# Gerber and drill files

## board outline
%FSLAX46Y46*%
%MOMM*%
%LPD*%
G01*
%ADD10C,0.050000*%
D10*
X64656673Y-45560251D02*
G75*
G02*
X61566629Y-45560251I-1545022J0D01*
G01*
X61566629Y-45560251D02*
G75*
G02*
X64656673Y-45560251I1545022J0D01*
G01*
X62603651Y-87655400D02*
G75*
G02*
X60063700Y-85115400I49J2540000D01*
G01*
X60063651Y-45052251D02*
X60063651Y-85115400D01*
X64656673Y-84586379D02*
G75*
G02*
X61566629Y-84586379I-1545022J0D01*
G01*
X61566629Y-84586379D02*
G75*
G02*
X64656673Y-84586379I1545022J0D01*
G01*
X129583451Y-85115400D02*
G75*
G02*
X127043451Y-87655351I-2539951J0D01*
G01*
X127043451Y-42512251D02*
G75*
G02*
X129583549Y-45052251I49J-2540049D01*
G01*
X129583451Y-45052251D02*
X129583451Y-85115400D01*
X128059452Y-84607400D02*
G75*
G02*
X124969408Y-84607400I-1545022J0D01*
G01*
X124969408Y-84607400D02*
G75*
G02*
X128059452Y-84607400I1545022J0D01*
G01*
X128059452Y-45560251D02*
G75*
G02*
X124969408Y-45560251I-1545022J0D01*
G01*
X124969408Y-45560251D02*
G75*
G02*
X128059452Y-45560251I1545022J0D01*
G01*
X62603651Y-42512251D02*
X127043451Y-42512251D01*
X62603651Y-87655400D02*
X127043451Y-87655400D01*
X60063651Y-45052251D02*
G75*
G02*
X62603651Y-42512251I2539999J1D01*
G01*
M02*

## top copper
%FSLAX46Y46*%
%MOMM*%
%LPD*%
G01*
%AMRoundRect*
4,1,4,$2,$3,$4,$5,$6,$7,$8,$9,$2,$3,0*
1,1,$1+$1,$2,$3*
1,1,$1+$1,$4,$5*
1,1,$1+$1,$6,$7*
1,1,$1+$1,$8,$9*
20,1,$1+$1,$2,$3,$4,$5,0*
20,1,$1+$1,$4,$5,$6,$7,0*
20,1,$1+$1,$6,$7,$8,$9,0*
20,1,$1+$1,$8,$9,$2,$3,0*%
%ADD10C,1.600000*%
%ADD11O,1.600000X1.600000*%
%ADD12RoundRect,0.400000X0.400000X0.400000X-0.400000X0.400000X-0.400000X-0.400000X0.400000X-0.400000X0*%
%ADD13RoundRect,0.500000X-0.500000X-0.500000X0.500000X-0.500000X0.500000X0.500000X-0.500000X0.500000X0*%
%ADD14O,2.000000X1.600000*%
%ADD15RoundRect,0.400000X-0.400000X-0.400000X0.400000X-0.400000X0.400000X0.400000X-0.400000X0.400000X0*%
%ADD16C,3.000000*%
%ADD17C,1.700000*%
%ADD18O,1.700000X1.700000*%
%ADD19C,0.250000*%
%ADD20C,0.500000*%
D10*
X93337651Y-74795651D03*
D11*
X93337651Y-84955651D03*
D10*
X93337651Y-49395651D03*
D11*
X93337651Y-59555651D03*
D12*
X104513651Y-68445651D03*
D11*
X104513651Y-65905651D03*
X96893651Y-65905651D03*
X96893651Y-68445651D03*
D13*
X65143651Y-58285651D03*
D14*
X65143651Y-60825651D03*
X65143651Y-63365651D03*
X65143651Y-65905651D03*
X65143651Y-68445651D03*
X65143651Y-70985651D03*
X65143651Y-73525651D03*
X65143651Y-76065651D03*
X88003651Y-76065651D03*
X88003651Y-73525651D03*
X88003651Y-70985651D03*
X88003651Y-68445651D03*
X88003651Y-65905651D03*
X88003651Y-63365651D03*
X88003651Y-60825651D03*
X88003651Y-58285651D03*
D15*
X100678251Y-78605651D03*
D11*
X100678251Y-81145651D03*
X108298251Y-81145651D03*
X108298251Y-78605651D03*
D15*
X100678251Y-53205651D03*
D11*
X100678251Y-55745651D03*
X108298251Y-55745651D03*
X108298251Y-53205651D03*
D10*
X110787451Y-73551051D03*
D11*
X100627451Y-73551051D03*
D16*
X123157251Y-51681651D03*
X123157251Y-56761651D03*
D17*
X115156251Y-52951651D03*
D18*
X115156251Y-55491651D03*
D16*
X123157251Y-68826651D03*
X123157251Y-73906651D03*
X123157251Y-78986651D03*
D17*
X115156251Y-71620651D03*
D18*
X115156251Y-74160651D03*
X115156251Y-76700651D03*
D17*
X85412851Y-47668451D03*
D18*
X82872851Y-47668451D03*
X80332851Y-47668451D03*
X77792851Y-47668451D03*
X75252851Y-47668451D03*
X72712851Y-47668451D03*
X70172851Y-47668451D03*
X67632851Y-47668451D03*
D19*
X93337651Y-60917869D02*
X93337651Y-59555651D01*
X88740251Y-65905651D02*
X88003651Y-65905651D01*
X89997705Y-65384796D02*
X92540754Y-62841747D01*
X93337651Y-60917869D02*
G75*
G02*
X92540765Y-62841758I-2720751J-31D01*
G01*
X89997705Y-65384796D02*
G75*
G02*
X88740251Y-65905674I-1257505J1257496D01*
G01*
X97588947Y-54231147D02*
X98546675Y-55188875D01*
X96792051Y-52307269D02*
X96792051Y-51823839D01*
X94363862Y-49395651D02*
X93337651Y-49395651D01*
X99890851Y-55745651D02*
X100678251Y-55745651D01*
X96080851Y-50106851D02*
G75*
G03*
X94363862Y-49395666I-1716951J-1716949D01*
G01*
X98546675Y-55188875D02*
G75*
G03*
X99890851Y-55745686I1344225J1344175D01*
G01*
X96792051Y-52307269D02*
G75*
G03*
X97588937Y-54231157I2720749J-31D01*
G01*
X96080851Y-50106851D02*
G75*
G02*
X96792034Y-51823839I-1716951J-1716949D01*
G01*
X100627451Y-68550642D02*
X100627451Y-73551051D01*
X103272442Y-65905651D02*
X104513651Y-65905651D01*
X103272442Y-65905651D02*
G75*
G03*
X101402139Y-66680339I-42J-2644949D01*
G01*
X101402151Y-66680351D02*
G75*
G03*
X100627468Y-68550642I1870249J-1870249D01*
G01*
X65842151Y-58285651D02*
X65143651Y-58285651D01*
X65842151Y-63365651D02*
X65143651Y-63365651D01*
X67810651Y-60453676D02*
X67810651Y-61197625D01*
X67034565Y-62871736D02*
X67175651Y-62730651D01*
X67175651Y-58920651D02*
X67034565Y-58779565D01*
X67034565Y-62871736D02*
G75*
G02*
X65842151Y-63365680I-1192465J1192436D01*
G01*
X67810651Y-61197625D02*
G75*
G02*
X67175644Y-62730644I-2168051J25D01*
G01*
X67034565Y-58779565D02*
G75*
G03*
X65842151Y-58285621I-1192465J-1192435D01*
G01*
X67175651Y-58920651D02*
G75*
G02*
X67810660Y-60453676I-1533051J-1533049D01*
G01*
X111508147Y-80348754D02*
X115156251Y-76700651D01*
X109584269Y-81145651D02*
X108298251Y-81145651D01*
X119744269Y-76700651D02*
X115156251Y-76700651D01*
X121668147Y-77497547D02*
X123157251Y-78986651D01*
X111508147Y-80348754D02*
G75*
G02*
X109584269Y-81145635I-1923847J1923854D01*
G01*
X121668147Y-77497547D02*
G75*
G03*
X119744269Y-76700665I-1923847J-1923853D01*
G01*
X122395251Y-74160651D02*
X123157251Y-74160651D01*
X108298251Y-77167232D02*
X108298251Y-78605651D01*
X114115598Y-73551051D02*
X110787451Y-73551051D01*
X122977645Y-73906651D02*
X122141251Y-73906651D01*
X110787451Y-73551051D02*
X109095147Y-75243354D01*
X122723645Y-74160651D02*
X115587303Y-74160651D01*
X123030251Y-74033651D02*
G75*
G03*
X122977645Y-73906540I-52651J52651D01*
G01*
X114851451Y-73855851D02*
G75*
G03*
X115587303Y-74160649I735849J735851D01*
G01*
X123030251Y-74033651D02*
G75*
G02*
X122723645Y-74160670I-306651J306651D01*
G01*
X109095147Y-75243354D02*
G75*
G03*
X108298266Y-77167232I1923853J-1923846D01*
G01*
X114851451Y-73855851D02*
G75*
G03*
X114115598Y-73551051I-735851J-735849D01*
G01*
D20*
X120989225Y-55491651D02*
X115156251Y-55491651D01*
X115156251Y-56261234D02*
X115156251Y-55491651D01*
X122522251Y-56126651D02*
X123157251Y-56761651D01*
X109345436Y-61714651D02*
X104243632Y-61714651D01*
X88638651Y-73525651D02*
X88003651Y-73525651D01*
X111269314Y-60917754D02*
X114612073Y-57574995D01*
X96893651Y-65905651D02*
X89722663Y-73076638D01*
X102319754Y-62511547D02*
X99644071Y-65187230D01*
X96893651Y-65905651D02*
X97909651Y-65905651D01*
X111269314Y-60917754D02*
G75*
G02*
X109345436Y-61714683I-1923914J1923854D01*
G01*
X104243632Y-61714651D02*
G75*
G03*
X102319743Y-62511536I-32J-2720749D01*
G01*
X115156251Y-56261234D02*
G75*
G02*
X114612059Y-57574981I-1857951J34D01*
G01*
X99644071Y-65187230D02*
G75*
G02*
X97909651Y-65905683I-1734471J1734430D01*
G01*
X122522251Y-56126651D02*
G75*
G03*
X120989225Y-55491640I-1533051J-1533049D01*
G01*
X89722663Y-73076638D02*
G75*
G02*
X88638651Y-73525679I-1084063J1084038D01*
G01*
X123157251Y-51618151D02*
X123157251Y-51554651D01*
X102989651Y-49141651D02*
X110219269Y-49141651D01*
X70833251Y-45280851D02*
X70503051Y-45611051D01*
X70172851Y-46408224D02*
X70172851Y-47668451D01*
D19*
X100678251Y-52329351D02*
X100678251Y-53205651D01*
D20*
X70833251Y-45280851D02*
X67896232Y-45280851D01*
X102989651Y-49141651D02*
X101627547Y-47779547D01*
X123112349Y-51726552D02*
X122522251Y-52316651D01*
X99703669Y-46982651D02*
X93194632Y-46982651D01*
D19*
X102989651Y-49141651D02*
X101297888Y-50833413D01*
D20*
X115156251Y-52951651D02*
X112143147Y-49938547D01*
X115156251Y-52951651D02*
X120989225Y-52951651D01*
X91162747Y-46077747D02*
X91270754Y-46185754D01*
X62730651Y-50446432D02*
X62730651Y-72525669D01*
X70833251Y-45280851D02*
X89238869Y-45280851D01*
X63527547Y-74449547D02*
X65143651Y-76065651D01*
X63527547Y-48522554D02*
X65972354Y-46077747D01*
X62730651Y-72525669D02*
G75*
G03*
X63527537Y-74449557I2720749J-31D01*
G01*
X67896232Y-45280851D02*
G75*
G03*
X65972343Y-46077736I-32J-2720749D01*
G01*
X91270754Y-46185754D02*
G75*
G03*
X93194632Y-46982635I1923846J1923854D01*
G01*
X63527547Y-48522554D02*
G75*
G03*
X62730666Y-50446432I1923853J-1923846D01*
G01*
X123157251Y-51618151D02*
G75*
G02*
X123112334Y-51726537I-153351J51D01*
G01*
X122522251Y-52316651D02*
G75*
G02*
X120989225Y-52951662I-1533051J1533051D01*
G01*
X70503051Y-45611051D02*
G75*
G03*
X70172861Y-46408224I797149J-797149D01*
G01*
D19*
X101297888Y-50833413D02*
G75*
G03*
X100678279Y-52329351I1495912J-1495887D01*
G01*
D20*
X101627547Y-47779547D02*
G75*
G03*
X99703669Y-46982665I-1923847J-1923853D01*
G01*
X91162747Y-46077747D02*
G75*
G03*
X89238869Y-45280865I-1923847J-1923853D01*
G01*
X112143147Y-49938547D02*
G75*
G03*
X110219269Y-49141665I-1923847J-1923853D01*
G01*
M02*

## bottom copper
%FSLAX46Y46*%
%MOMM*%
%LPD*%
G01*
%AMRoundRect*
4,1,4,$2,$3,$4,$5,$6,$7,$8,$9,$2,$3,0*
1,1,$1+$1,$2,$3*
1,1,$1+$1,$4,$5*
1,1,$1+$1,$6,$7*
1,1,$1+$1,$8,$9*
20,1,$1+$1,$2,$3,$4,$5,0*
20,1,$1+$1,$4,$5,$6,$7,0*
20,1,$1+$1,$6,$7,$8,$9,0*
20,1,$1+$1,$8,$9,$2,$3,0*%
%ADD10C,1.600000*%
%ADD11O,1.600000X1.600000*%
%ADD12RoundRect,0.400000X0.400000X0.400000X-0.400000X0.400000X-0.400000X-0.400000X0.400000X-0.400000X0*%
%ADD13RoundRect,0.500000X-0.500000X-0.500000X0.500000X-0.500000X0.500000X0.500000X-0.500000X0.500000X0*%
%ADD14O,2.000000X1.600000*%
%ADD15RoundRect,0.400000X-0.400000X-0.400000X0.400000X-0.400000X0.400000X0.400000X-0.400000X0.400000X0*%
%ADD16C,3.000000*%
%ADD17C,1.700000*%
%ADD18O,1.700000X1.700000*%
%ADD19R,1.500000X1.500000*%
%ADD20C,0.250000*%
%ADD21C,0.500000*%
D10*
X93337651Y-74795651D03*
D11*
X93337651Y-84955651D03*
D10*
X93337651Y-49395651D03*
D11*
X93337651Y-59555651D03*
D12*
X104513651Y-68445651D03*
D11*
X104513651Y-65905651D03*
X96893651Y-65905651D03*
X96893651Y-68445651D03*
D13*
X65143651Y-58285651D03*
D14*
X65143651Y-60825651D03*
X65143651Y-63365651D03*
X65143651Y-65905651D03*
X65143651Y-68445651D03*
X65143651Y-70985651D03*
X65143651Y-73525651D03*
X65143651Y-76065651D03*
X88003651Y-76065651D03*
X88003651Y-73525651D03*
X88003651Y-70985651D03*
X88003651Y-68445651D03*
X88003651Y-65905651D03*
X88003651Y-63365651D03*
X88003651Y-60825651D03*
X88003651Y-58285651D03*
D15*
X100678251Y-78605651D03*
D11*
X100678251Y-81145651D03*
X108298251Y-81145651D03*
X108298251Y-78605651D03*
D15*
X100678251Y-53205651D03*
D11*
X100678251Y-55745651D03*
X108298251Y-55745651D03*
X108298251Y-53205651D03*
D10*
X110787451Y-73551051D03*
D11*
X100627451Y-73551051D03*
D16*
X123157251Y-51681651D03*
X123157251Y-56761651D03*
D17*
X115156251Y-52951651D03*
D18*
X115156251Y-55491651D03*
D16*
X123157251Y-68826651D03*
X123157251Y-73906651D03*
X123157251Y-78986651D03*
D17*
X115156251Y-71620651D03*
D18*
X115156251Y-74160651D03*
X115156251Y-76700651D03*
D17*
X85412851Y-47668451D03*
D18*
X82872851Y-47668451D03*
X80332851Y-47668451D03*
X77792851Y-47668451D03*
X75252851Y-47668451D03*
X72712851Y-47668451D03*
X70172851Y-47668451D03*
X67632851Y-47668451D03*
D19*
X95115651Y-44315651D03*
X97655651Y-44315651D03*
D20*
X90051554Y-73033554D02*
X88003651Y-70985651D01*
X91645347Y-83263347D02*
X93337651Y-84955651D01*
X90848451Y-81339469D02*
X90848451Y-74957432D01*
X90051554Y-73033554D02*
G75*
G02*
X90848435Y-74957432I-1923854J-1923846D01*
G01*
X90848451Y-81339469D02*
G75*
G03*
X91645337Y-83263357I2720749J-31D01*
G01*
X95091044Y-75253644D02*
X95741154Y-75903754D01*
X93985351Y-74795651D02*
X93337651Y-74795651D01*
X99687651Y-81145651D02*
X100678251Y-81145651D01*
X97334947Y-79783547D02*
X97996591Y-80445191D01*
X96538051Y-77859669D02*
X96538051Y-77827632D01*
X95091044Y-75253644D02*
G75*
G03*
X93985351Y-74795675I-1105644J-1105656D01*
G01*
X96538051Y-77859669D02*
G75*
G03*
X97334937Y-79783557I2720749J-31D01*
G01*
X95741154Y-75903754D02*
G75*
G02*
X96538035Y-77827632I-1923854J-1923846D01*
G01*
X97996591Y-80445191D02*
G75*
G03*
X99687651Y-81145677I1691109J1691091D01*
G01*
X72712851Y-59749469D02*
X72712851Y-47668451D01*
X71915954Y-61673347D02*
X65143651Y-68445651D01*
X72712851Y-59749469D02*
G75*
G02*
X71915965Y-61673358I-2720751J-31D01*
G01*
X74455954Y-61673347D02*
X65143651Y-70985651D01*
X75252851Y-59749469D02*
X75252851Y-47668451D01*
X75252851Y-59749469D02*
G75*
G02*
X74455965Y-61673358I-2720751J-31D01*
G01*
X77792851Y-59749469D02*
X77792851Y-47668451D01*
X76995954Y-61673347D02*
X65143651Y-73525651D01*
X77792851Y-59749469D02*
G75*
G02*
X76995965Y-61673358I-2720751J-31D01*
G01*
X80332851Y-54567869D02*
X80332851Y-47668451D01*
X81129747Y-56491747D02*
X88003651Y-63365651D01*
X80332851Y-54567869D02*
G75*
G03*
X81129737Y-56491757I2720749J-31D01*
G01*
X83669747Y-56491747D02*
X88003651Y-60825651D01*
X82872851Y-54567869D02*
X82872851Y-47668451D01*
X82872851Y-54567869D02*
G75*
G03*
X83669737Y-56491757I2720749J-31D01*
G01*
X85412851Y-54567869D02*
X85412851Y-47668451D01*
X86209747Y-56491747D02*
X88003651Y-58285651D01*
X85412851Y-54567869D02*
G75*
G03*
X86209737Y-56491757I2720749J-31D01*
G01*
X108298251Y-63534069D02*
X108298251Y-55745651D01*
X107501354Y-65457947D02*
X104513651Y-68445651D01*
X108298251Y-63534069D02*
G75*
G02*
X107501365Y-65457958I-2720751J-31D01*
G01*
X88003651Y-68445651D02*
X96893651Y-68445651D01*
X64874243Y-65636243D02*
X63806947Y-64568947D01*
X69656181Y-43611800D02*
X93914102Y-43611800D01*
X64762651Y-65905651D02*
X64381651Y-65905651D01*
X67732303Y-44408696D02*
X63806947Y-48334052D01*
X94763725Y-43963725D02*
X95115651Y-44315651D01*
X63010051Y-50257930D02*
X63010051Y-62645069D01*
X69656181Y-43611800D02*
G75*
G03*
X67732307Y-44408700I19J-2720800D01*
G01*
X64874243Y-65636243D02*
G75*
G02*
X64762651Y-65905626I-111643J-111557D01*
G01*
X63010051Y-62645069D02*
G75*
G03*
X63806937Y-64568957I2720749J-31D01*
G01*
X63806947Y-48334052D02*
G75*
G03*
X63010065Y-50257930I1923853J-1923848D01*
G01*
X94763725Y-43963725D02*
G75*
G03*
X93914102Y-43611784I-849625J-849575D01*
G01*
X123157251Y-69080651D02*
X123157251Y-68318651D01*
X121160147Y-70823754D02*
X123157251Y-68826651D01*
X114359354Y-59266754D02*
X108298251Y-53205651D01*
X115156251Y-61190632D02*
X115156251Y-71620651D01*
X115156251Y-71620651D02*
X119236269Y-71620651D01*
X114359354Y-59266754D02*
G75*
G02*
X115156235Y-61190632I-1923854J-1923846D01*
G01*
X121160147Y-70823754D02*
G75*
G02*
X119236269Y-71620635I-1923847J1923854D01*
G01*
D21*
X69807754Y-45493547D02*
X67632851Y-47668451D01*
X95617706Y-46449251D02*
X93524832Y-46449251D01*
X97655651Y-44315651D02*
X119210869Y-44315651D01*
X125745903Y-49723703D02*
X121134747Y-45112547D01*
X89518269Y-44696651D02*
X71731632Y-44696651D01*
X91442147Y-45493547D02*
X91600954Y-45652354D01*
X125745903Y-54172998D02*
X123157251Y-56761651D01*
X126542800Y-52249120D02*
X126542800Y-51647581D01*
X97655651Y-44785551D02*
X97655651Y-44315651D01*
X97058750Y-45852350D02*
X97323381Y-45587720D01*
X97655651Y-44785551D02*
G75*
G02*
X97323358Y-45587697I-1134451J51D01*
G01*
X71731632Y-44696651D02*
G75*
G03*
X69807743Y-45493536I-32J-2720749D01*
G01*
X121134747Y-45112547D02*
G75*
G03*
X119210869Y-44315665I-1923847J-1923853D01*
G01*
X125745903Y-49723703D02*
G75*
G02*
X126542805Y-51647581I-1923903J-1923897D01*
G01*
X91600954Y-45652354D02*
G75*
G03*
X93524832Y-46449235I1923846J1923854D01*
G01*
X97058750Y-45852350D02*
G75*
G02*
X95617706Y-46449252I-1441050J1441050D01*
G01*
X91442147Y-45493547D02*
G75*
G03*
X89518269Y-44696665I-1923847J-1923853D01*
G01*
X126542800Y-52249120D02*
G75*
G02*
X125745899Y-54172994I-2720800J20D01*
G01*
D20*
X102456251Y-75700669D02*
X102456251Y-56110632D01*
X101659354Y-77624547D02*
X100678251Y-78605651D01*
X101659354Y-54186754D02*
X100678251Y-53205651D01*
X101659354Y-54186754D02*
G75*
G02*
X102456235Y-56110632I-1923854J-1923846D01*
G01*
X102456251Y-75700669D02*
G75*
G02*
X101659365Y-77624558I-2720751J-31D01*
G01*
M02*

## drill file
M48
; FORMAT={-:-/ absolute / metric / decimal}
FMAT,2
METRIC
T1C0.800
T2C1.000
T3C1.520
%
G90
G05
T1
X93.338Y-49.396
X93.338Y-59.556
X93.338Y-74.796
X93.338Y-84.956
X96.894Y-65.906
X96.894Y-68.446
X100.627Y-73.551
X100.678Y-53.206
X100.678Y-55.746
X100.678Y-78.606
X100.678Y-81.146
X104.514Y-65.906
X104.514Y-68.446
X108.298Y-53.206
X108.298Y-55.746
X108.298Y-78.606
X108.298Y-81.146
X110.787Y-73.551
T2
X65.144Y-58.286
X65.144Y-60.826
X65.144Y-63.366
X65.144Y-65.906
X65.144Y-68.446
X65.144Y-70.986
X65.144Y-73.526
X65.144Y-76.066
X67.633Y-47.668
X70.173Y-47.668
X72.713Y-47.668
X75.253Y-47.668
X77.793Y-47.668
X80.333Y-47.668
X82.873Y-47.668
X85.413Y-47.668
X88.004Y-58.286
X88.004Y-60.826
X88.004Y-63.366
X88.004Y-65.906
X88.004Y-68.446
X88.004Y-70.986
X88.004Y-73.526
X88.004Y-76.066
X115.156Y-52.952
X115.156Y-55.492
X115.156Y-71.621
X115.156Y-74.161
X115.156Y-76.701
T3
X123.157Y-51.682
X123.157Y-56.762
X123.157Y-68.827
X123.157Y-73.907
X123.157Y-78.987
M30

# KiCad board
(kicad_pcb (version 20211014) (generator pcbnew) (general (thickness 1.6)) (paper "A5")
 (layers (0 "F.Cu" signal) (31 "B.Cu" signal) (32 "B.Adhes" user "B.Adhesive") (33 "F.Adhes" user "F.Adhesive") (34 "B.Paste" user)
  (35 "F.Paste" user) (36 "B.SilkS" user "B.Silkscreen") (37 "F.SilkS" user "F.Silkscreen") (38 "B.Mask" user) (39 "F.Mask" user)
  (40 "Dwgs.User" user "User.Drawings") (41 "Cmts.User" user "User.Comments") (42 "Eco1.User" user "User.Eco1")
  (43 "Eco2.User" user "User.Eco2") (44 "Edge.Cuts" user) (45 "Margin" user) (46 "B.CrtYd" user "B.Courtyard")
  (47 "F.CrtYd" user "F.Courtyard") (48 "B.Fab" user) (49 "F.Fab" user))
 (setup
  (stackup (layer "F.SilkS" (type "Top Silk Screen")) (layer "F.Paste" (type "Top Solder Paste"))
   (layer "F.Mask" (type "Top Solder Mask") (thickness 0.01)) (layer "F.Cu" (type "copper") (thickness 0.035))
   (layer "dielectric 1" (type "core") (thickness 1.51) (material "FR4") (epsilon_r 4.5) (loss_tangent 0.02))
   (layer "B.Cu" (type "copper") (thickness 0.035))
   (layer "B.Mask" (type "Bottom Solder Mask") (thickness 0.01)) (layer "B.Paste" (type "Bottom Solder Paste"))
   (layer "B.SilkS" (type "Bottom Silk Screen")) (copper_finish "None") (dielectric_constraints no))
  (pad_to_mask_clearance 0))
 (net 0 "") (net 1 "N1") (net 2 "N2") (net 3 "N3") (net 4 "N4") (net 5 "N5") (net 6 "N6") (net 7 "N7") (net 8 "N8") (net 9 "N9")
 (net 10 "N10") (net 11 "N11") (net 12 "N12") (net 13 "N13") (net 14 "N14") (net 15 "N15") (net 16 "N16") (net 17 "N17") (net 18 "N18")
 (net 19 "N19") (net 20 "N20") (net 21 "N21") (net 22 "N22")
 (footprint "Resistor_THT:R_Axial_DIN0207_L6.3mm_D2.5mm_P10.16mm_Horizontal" (layer "F.Cu") (at 93.337651 74.795651 -90)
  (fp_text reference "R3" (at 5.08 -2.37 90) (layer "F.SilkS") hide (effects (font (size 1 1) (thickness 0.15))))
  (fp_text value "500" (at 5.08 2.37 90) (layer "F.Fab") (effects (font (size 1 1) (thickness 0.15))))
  (pad "1" thru_hole circle locked (at 0 0 270) (size 1.6 1.6) (drill 0.8) (layers *.Cu *.Mask) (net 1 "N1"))
  (pad "2" thru_hole oval locked (at 10.16 0 270) (size 1.6 1.6) (drill 0.8) (layers *.Cu *.Mask) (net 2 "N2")))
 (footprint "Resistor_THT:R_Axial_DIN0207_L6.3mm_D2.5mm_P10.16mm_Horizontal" (layer "F.Cu") (at 93.337651 49.395651 -90)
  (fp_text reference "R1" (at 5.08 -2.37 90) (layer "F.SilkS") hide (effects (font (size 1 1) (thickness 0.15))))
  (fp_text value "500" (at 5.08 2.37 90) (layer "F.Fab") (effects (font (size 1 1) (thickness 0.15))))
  (pad "1" thru_hole circle locked (at 0 0 270) (size 1.6 1.6) (drill 0.8) (layers *.Cu *.Mask) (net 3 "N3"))
  (pad "2" thru_hole oval locked (at 10.16 0 270) (size 1.6 1.6) (drill 0.8) (layers *.Cu *.Mask) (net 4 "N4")))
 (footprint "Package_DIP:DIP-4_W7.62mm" (layer "F.Cu") (at 104.513651 68.445651 180)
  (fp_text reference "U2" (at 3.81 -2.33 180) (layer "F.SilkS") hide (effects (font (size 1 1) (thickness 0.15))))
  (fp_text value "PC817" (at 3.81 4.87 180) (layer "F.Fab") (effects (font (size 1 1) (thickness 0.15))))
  (pad "1" thru_hole roundrect locked (at 0 0 180) (size 1.6 1.6) (drill 0.8) (layers *.Cu *.Mask) (roundrect_rratio 0.25) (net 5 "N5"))
  (pad "2" thru_hole oval locked (at 0 2.54 180) (size 1.6 1.6) (drill 0.8) (layers *.Cu *.Mask) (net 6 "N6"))
  (pad "3" thru_hole oval locked (at 7.62 2.54 180) (size 1.6 1.6) (drill 0.8) (layers *.Cu *.Mask) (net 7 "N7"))
  (pad "4" thru_hole oval locked (at 7.62 0 180) (size 1.6 1.6) (drill 0.8) (layers *.Cu *.Mask) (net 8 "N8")))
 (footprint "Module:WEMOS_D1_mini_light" (layer "F.Cu") (at 65.143651 58.285651)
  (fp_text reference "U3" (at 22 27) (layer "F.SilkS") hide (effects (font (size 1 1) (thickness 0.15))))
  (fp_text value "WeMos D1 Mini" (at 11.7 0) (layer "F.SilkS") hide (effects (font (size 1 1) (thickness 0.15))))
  (pad "1" thru_hole roundrect locked (at 0 0) (size 2 2) (drill 1) (layers *.Cu *.Mask) (roundrect_rratio 0.25) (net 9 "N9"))
  (pad "2" thru_hole oval locked (at 0 2.54) (size 2 1.6) (drill 1) (layers *.Cu *.Mask) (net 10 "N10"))
  (pad "3" thru_hole oval locked (at 0 5.08) (size 2 1.6) (drill 1) (layers *.Cu *.Mask) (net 9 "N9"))
  (pad "4" thru_hole oval locked (at 0 7.62) (size 2 1.6) (drill 1) (layers *.Cu *.Mask) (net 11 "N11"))
  (pad "5" thru_hole oval locked (at 0 10.16) (size 2 1.6) (drill 1) (layers *.Cu *.Mask) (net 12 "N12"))
  (pad "6" thru_hole oval locked (at 0 12.7) (size 2 1.6) (drill 1) (layers *.Cu *.Mask) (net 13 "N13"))
  (pad "7" thru_hole oval locked (at 0 15.24) (size 2 1.6) (drill 1) (layers *.Cu *.Mask) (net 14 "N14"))
  (pad "8" thru_hole oval locked (at 0 17.78) (size 2 1.6) (drill 1) (layers *.Cu *.Mask) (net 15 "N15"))
  (pad "9" thru_hole oval locked (at 22.86 17.78) (size 2 1.6) (drill 1) (layers *.Cu *.Mask) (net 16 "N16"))
  (pad "10" thru_hole oval locked (at 22.86 15.24) (size 2 1.6) (drill 1) (layers *.Cu *.Mask) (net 7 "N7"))
  (pad "11" thru_hole oval locked (at 22.86 12.7) (size 2 1.6) (drill 1) (layers *.Cu *.Mask) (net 2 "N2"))
  (pad "12" thru_hole oval locked (at 22.86 10.16) (size 2 1.6) (drill 1) (layers *.Cu *.Mask) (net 8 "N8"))
  (pad "13" thru_hole oval locked (at 22.86 7.62) (size 2 1.6) (drill 1) (layers *.Cu *.Mask) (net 4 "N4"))
  (pad "14" thru_hole oval locked (at 22.86 5.08) (size 2 1.6) (drill 1) (layers *.Cu *.Mask) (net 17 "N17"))
  (pad "15" thru_hole oval locked (at 22.86 2.54) (size 2 1.6) (drill 1) (layers *.Cu *.Mask) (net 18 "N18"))
  (pad "16" thru_hole oval locked (at 22.86 0) (size 2 1.6) (drill 1) (layers *.Cu *.Mask) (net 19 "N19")))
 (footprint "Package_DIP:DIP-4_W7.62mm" (layer "F.Cu") (at 100.678251 78.605651)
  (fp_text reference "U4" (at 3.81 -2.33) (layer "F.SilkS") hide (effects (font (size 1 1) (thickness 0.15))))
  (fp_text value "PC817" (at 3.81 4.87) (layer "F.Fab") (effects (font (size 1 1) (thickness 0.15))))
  (pad "1" thru_hole roundrect locked (at 0 0) (size 1.6 1.6) (drill 0.8) (layers *.Cu *.Mask) (roundrect_rratio 0.25) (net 15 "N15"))
  (pad "2" thru_hole oval locked (at 0 2.54) (size 1.6 1.6) (drill 0.8) (layers *.Cu *.Mask) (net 1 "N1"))
  (pad "3" thru_hole oval locked (at 7.62 2.54) (size 1.6 1.6) (drill 0.8) (layers *.Cu *.Mask) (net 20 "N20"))
  (pad "4" thru_hole oval locked (at 7.62 0) (size 1.6 1.6) (drill 0.8) (layers *.Cu *.Mask) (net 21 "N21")))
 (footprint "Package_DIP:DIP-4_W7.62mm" (layer "F.Cu") (at 100.678251 53.205651)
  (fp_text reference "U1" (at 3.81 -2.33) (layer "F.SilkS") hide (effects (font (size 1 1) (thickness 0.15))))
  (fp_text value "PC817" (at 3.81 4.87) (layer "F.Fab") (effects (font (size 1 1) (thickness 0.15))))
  (pad "1" thru_hole roundrect locked (at 0 0) (size 1.6 1.6) (drill 0.8) (layers *.Cu *.Mask) (roundrect_rratio 0.25) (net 15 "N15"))
  (pad "2" thru_hole oval locked (at 0 2.54) (size 1.6 1.6) (drill 0.8) (layers *.Cu *.Mask) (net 3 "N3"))
  (pad "3" thru_hole oval locked (at 7.62 2.54) (size 1.6 1.6) (drill 0.8) (layers *.Cu *.Mask) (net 5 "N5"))
  (pad "4" thru_hole oval locked (at 7.62 0) (size 1.6 1.6) (drill 0.8) (layers *.Cu *.Mask) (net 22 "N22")))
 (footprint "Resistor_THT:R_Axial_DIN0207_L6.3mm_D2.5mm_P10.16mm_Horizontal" (layer "F.Cu") (at 110.787451 73.551051 180)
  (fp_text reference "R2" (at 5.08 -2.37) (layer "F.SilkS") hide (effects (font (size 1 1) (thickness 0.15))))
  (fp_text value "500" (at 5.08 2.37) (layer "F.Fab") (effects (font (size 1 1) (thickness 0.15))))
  (pad "1" thru_hole circle locked (at 0 0 180) (size 1.6 1.6) (drill 0.8) (layers *.Cu *.Mask) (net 21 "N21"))
  (pad "2" thru_hole oval locked (at 10.16 0 180) (size 1.6 1.6) (drill 0.8) (layers *.Cu *.Mask) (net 6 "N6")))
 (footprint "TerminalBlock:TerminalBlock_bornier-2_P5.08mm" (layer "F.Cu") (at 123.157251 51.681651 -90)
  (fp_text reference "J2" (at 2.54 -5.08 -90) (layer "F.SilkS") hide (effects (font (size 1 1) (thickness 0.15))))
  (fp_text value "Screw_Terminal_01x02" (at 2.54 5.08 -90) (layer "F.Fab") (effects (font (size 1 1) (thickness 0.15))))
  (pad "1" thru_hole circle locked (at 0 0 270) (size 3 3) (drill 1.52) (layers *.Cu *.Mask) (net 15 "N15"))
  (pad "2" thru_hole circle locked (at 5.08 0 270) (size 3 3) (drill 1.52) (layers *.Cu *.Mask) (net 7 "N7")))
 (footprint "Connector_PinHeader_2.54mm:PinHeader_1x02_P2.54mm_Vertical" (layer "F.Cu") (at 115.156251 52.951651)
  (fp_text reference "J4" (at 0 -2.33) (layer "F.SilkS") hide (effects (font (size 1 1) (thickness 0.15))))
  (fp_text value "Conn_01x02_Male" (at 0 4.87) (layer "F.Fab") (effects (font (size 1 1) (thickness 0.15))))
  (pad "1" thru_hole circle locked (at 0 0) (size 1.7 1.7) (drill 1) (layers *.Cu *.Mask) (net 15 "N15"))
  (pad "2" thru_hole oval locked (at 0 2.54) (size 1.7 1.7) (drill 1) (layers *.Cu *.Mask) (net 7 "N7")))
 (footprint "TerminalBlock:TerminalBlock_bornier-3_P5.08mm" (layer "F.Cu") (at 123.157251 68.826651 -90)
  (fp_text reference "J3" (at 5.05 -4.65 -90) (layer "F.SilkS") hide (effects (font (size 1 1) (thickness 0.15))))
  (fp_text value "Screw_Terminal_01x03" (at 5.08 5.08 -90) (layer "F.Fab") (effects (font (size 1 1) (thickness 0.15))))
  (pad "1" thru_hole circle locked (at 0 0 270) (size 3 3) (drill 1.52) (layers *.Cu *.Mask) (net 22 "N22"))
  (pad "2" thru_hole circle locked (at 5.08 0 270) (size 3 3) (drill 1.52) (layers *.Cu *.Mask) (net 21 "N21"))
  (pad "3" thru_hole circle locked (at 10.16 0 270) (size 3 3) (drill 1.52) (layers *.Cu *.Mask) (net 20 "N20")))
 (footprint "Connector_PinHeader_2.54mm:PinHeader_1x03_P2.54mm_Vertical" (layer "F.Cu") (at 115.156251 71.620651)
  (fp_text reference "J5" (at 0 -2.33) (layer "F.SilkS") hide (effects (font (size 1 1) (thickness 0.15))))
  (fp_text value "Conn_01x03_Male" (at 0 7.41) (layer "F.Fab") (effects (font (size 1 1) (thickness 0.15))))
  (pad "1" thru_hole circle locked (at 0 0) (size 1.7 1.7) (drill 1) (layers *.Cu *.Mask) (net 22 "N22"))
  (pad "2" thru_hole oval locked (at 0 2.54) (size 1.7 1.7) (drill 1) (layers *.Cu *.Mask) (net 21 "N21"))
  (pad "3" thru_hole oval locked (at 0 5.08) (size 1.7 1.7) (drill 1) (layers *.Cu *.Mask) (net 20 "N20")))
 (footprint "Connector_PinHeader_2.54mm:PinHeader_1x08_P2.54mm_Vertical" (layer "F.Cu") (at 85.412851 47.668451 -90)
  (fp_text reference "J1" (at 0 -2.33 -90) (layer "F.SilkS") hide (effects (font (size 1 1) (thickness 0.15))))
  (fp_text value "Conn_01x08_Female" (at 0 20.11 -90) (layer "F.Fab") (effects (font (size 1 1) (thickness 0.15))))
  (pad "1" thru_hole circle locked (at 0 0 270) (size 1.7 1.7) (drill 1) (layers *.Cu *.Mask) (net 19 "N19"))
  (pad "2" thru_hole oval locked (at 0 2.54 270) (size 1.7 1.7) (drill 1) (layers *.Cu *.Mask) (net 18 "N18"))
  (pad "3" thru_hole oval locked (at 0 5.08 270) (size 1.7 1.7) (drill 1) (layers *.Cu *.Mask) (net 17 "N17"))
  (pad "4" thru_hole oval locked (at 0 7.62 270) (size 1.7 1.7) (drill 1) (layers *.Cu *.Mask) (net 14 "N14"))
  (pad "5" thru_hole oval locked (at 0 10.16 270) (size 1.7 1.7) (drill 1) (layers *.Cu *.Mask) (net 13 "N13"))
  (pad "6" thru_hole oval locked (at 0 12.7 270) (size 1.7 1.7) (drill 1) (layers *.Cu *.Mask) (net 12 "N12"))
  (pad "7" thru_hole oval locked (at 0 15.24 270) (size 1.7 1.7) (drill 1) (layers *.Cu *.Mask) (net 15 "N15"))
  (pad "8" thru_hole oval locked (at 0 17.78 270) (size 1.7 1.7) (drill 1) (layers *.Cu *.Mask) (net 7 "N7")))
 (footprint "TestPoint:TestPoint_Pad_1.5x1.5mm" (layer "B.Cu") (at 95.115651 44.315651 180)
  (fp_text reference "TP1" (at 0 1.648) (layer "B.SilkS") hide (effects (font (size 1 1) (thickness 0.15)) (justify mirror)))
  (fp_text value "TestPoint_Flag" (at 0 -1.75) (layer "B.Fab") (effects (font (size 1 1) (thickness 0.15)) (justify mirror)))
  (pad "1" smd rect locked (at 0 0 180) (size 1.5 1.5) (layers "B.Cu" "B.Mask") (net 11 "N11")))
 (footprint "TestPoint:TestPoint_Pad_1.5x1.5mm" (layer "B.Cu") (at 97.655651 44.315651 180)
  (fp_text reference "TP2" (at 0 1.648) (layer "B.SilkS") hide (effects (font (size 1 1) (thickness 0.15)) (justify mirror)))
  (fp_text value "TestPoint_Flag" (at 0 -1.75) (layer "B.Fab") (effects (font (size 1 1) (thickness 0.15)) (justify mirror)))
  (pad "1" smd rect locked (at 0 0 180) (size 1.5 1.5) (layers "B.Cu" "B.Mask") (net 7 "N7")))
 (gr_circle (center 63.111651 45.560251) (end 64.635651 45.306251) (layer "Edge.Cuts") (width 0.05) (fill none))
 (gr_arc (start 62.603651 87.6554) (mid 60.8076 86.911451) (end 60.063651 85.1154) (layer "Edge.Cuts") (width 0.05))
 (gr_line (start 60.063651 45.052251) (end 60.063651 85.1154) (layer "Edge.Cuts") (width 0.05))
 (gr_circle (center 63.111651 84.586379) (end 64.635651 84.332379) (layer "Edge.Cuts") (width 0.05) (fill none))
 (gr_arc (start 129.583451 85.1154) (mid 128.839502 86.911451) (end 127.043451 87.6554) (layer "Edge.Cuts") (width 0.05))
 (gr_arc (start 127.043451 42.512251) (mid 128.839502 43.2562) (end 129.583451 45.052251) (layer "Edge.Cuts") (width 0.05))
 (gr_line (start 129.583451 45.052251) (end 129.583451 85.1154) (layer "Edge.Cuts") (width 0.05))
 (gr_circle (center 126.51443 84.6074) (end 128.03843 84.3534) (layer "Edge.Cuts") (width 0.05) (fill none))
 (gr_circle (center 126.51443 45.560251) (end 128.03843 45.306251) (layer "Edge.Cuts") (width 0.05) (fill none))
 (gr_line (start 62.603651 42.512251) (end 127.043451 42.512251) (layer "Edge.Cuts") (width 0.05))
 (gr_line (start 62.603651 87.6554) (end 127.043451 87.6554) (layer "Edge.Cuts") (width 0.05))
 (gr_arc (start 60.063651 45.052251) (mid 60.8076 43.2562) (end 62.603651 42.512251) (layer "Edge.Cuts") (width 0.05))
 (segment (start 93.337651 60.917869) (end 93.337651 59.555651) (width 0.25) (layer "F.Cu") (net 4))
 (segment (start 88.740251 65.905651) (end 88.003651 65.905651) (width 0.25) (layer "F.Cu") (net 4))
 (segment (start 89.997705 65.384796) (end 92.540754 62.841747) (width 0.25) (layer "F.Cu") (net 4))
 (arc (start 93.337651 60.917869) (mid 93.130544 61.959064) (end 92.540754 62.841747) (width 0.25) (layer "F.Cu") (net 4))
 (arc (start 89.997705 65.384796) (mid 89.42078 65.770285) (end 88.740251 65.905651) (width 0.25) (layer "F.Cu") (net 4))
 (segment (start 97.588947 54.231147) (end 98.546675 55.188875) (width 0.25) (layer "F.Cu") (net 3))
 (segment (start 96.792051 52.307269) (end 96.792051 51.823839) (width 0.25) (layer "F.Cu") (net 3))
 (segment (start 94.363862 49.395651) (end 93.337651 49.395651) (width 0.25) (layer "F.Cu") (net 3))
 (segment (start 99.890851 55.745651) (end 100.678251 55.745651) (width 0.25) (layer "F.Cu") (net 3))
 (arc (start 96.080851 50.106851) (mid 95.293089 49.580485) (end 94.363862 49.395651) (width 0.25) (layer "F.Cu") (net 3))
 (arc (start 98.546675 55.188875) (mid 99.163388 55.600949) (end 99.890851 55.745651) (width 0.25) (layer "F.Cu") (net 3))
 (arc (start 96.792051 52.307269) (mid 96.999157 53.348464) (end 97.588947 54.231147) (width 0.25) (layer "F.Cu") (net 3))
 (arc (start 96.080851 50.106851) (mid 96.607216 50.894611) (end 96.792051 51.823839) (width 0.25) (layer "F.Cu") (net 3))
 (segment (start 100.627451 68.550642) (end 100.627451 73.551051) (width 0.25) (layer "F.Cu") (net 6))
 (segment (start 103.272442 65.905651) (end 104.513651 65.905651) (width 0.25) (layer "F.Cu") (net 6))
 (arc (start 103.272442 65.905651) (mid 102.260247 66.106988) (end 101.402151 66.680351) (width 0.25) (layer "F.Cu") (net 6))
 (arc (start 101.402151 66.680351) (mid 100.828788 67.538447) (end 100.627451 68.550642) (width 0.25) (layer "F.Cu") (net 6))
 (segment (start 90.051554 73.033554) (end 88.003651 70.985651) (width 0.25) (layer "B.Cu") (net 2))
 (segment (start 91.645347 83.263347) (end 93.337651 84.955651) (width 0.25) (layer "B.Cu") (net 2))
 (segment (start 90.848451 81.339469) (end 90.848451 74.957432) (width 0.25) (layer "B.Cu") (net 2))
 (arc (start 90.051554 73.033554) (mid 90.641344 73.916237) (end 90.848451 74.957432) (width 0.25) (layer "B.Cu") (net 2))
 (arc (start 90.848451 81.339469) (mid 91.055557 82.380664) (end 91.645347 83.263347) (width 0.25) (layer "B.Cu") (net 2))
 (segment (start 95.091044 75.253644) (end 95.741154 75.903754) (width 0.25) (layer "B.Cu") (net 1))
 (segment (start 93.985351 74.795651) (end 93.337651 74.795651) (width 0.25) (layer "B.Cu") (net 1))
 (segment (start 99.687651 81.145651) (end 100.678251 81.145651) (width 0.25) (layer "B.Cu") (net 1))
 (segment (start 97.334947 79.783547) (end 97.996591 80.445191) (width 0.25) (layer "B.Cu") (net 1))
 (segment (start 96.538051 77.859669) (end 96.538051 77.827632) (width 0.25) (layer "B.Cu") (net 1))
 (arc (start 95.091044 75.253644) (mid 94.583747 74.914679) (end 93.985351 74.795651) (width 0.25) (layer "B.Cu") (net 1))
 (arc (start 96.538051 77.859669) (mid 96.745157 78.900864) (end 97.334947 79.783547) (width 0.25) (layer "B.Cu") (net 1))
 (arc (start 95.741154 75.903754) (mid 96.330944 76.786437) (end 96.538051 77.827632) (width 0.25) (layer "B.Cu") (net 1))
 (arc (start 97.996591 80.445191) (mid 98.772455 80.963607) (end 99.687651 81.145651) (width 0.25) (layer "B.Cu") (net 1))
 (segment (start 72.712851 59.749469) (end 72.712851 47.668451) (width 0.25) (layer "B.Cu") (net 12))
 (segment (start 71.915954 61.673347) (end 65.143651 68.445651) (width 0.25) (layer "B.Cu") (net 12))
 (arc (start 72.712851 59.749469) (mid 72.505744 60.790664) (end 71.915954 61.673347) (width 0.25) (layer "B.Cu") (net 12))
 (segment (start 74.455954 61.673347) (end 65.143651 70.985651) (width 0.25) (layer "B.Cu") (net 13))
 (segment (start 75.252851 59.749469) (end 75.252851 47.668451) (width 0.25) (layer "B.Cu") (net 13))
 (arc (start 75.252851 59.749469) (mid 75.045744 60.790664) (end 74.455954 61.673347) (width 0.25) (layer "B.Cu") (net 13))
 (segment (start 77.792851 59.749469) (end 77.792851 47.668451) (width 0.25) (layer "B.Cu") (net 14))
 (segment (start 76.995954 61.673347) (end 65.143651 73.525651) (width 0.25) (layer "B.Cu") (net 14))
 (arc (start 77.792851 59.749469) (mid 77.585744 60.790664) (end 76.995954 61.673347) (width 0.25) (layer "B.Cu") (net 14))
 (segment (start 80.332851 54.567869) (end 80.332851 47.668451) (width 0.25) (layer "B.Cu") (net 17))
 (segment (start 81.129747 56.491747) (end 88.003651 63.365651) (width 0.25) (layer "B.Cu") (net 17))
 (arc (start 80.332851 54.567869) (mid 80.539957 55.609064) (end 81.129747 56.491747) (width 0.25) (layer "B.Cu") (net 17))
 (segment (start 83.669747 56.491747) (end 88.003651 60.825651) (width 0.25) (layer "B.Cu") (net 18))
 (segment (start 82.872851 54.567869) (end 82.872851 47.668451) (width 0.25) (layer "B.Cu") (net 18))
 (arc (start 82.872851 54.567869) (mid 83.079957 55.609064) (end 83.669747 56.491747) (width 0.25) (layer "B.Cu") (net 18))
 (segment (start 85.412851 54.567869) (end 85.412851 47.668451) (width 0.25) (layer "B.Cu") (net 19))
 (segment (start 86.209747 56.491747) (end 88.003651 58.285651) (width 0.25) (layer "B.Cu") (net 19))
 (arc (start 85.412851 54.567869) (mid 85.619957 55.609064) (end 86.209747 56.491747) (width 0.25) (layer "B.Cu") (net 19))
 (segment (start 108.298251 63.534069) (end 108.298251 55.745651) (width 0.25) (layer "B.Cu") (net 5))
 (segment (start 107.501354 65.457947) (end 104.513651 68.445651) (width 0.25) (layer "B.Cu") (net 5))
 (arc (start 108.298251 63.534069) (mid 108.091144 64.575264) (end 107.501354 65.457947) (width 0.25) (layer "B.Cu") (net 5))
 (segment (start 88.003651 68.445651) (end 96.893651 68.445651) (width 0.25) (layer "B.Cu") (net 8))
 (segment (start 65.842151 58.285651) (end 65.143651 58.285651) (width 0.25) (layer "F.Cu") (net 9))
 (segment (start 65.842151 63.365651) (end 65.143651 63.365651) (width 0.25) (layer "F.Cu") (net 9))
 (segment (start 67.810651 60.453676) (end 67.810651 61.197625) (width 0.25) (layer "F.Cu") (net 9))
 (segment (start 67.034565 62.871736) (end 67.175651 62.730651) (width 0.25) (layer "F.Cu") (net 9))
 (segment (start 67.175651 58.920651) (end 67.034565 58.779565) (width 0.25) (layer "F.Cu") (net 9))
 (arc (start 67.034565 62.871736) (mid 66.48748 63.237286) (end 65.842151 63.365651) (width 0.25) (layer "F.Cu") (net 9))
 (arc (start 67.810651 61.197625) (mid 67.645619 62.027292) (end 67.175651 62.730651) (width 0.25) (layer "F.Cu") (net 9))
 (arc (start 67.034565 58.779565) (mid 66.48748 58.414015) (end 65.842151 58.285651) (width 0.25) (layer "F.Cu") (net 9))
 (arc (start 67.175651 58.920651) (mid 67.645619 59.624008) (end 67.810651 60.453676) (width 0.25) (layer "F.Cu") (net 9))
 (segment (start 64.874243 65.636243) (end 63.806947 64.568947) (width 0.25) (layer "B.Cu") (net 11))
 (segment (start 69.656181 43.6118) (end 93.914102 43.6118) (width 0.25) (layer "B.Cu") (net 11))
 (segment (start 64.762651 65.905651) (end 64.381651 65.905651) (width 0.25) (layer "B.Cu") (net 11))
 (segment (start 67.732303 44.408696) (end 63.806947 48.334052) (width 0.25) (layer "B.Cu") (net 11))
 (segment (start 94.763725 43.963725) (end 95.115651 44.315651) (width 0.25) (layer "B.Cu") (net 11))
 (segment (start 63.010051 50.25793) (end 63.010051 62.645069) (width 0.25) (layer "B.Cu") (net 11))
 (arc (start 69.656181 43.6118) (mid 68.614986 43.818906) (end 67.732303 44.408696) (width 0.25) (layer "B.Cu") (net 11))
 (arc (start 64.874243 65.636243) (mid 64.908453 65.808228) (end 64.762651 65.905651) (width 0.25) (layer "B.Cu") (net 11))
 (arc (start 63.010051 62.645069) (mid 63.217157 63.686264) (end 63.806947 64.568947) (width 0.25) (layer "B.Cu") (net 11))
 (arc (start 63.806947 48.334052) (mid 63.217157 49.216735) (end 63.010051 50.25793) (width 0.25) (layer "B.Cu") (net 11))
 (arc (start 94.763725 43.963725) (mid 94.373914 43.703262) (end 93.914102 43.6118) (width 0.25) (layer "B.Cu") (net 11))
 (segment (start 111.508147 80.348754) (end 115.156251 76.700651) (width 0.25) (layer "F.Cu") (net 20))
 (segment (start 109.584269 81.145651) (end 108.298251 81.145651) (width 0.25) (layer "F.Cu") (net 20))
 (segment (start 119.744269 76.700651) (end 115.156251 76.700651) (width 0.25) (layer "F.Cu") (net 20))
 (segment (start 121.668147 77.497547) (end 123.157251 78.986651) (width 0.25) (layer "F.Cu") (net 20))
 (arc (start 111.508147 80.348754) (mid 110.625464 80.938544) (end 109.584269 81.145651) (width 0.25) (layer "F.Cu") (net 20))
 (arc (start 121.668147 77.497547) (mid 120.785464 76.907757) (end 119.744269 76.700651) (width 0.25) (layer "F.Cu") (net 20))
 (segment (start 122.395251 74.160651) (end 123.157251 74.160651) (width 0.25) (layer "F.Cu") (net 21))
 (segment (start 108.298251 77.167232) (end 108.298251 78.605651) (width 0.25) (layer "F.Cu") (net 21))
 (segment (start 114.115598 73.551051) (end 110.787451 73.551051) (width 0.25) (layer "F.Cu") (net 21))
 (segment (start 122.977645 73.906651) (end 122.141251 73.906651) (width 0.25) (layer "F.Cu") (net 21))
 (segment (start 110.787451 73.551051) (end 109.095147 75.243354) (width 0.25) (layer "F.Cu") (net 21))
 (segment (start 122.723645 74.160651) (end 115.587303 74.160651) (width 0.25) (layer "F.Cu") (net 21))
 (arc (start 123.030251 74.033651) (mid 123.046377 73.952576) (end 122.977645 73.906651) (width 0.25) (layer "F.Cu") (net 21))
 (arc (start 114.851451 73.855851) (mid 115.189062 74.081436) (end 115.587303 74.160651) (width 0.25) (layer "F.Cu") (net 21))
 (arc (start 123.030251 74.033651) (mid 122.889579 74.127644) (end 122.723645 74.160651) (width 0.25) (layer "F.Cu") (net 21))
 (arc (start 109.095147 75.243354) (mid 108.505357 76.126037) (end 108.298251 77.167232) (width 0.25) (layer "F.Cu") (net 21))
 (arc (start 114.851451 73.855851) (mid 114.513838 73.630265) (end 114.115598 73.551051) (width 0.25) (layer "F.Cu") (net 21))
 (segment (start 123.157251 69.080651) (end 123.157251 68.318651) (width 0.25) (layer "B.Cu") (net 22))
 (segment (start 121.160147 70.823754) (end 123.157251 68.826651) (width 0.25) (layer "B.Cu") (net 22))
 (segment (start 114.359354 59.266754) (end 108.298251 53.205651) (width 0.25) (layer "B.Cu") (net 22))
 (segment (start 115.156251 61.190632) (end 115.156251 71.620651) (width 0.25) (layer "B.Cu") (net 22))
 (segment (start 115.156251 71.620651) (end 119.236269 71.620651) (width 0.25) (layer "B.Cu") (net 22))
 (arc (start 114.359354 59.266754) (mid 114.949144 60.149437) (end 115.156251 61.190632) (width 0.25) (layer "B.Cu") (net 22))
 (arc (start 121.160147 70.823754) (mid 120.277464 71.413544) (end 119.236269 71.620651) (width 0.25) (layer "B.Cu") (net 22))
 (segment (start 120.989225 55.491651) (end 115.156251 55.491651) (width 0.5) (layer "F.Cu") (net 7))
 (segment (start 115.156251 56.261234) (end 115.156251 55.491651) (width 0.5) (layer "F.Cu") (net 7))
 (segment (start 122.522251 56.126651) (end 123.157251 56.761651) (width 0.5) (layer "F.Cu") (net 7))
 (segment (start 109.345436 61.714651) (end 104.243632 61.714651) (width 0.5) (layer "F.Cu") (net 7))
 (segment (start 88.638651 73.525651) (end 88.003651 73.525651) (width 0.5) (layer "F.Cu") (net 7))
 (segment (start 111.269314 60.917754) (end 114.612073 57.574995) (width 0.5) (layer "F.Cu") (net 7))
 (segment (start 96.893651 65.905651) (end 89.722663 73.076638) (width 0.5) (layer "F.Cu") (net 7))
 (segment (start 102.319754 62.511547) (end 99.644071 65.18723) (width 0.5) (layer "F.Cu") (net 7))
 (segment (start 96.893651 65.905651) (end 97.909651 65.905651) (width 0.5) (layer "F.Cu") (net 7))
 (arc (start 111.269314 60.917754) (mid 110.386631 61.507544) (end 109.345436 61.714651) (width 0.5) (layer "F.Cu") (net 7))
 (arc (start 104.243632 61.714651) (mid 103.202437 61.921757) (end 102.319754 62.511547) (width 0.5) (layer "F.Cu") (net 7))
 (arc (start 115.156251 56.261234) (mid 115.014823 56.972236) (end 114.612073 57.574995) (width 0.5) (layer "F.Cu") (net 7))
 (arc (start 99.644071 65.18723) (mid 98.848312 65.718939) (end 97.909651 65.905651) (width 0.5) (layer "F.Cu") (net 7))
 (arc (start 122.522251 56.126651) (mid 121.818892 55.656682) (end 120.989225 55.491651) (width 0.5) (layer "F.Cu") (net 7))
 (arc (start 89.722663 73.076638) (mid 89.225314 73.408956) (end 88.638651 73.525651) (width 0.5) (layer "F.Cu") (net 7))
 (segment (start 69.807754 45.493547) (end 67.632851 47.668451) (width 0.5) (layer "B.Cu") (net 7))
 (segment (start 95.617706 46.449251) (end 93.524832 46.449251) (width 0.5) (layer "B.Cu") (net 7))
 (segment (start 97.655651 44.315651) (end 119.210869 44.315651) (width 0.5) (layer "B.Cu") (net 7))
 (segment (start 125.745903 49.723703) (end 121.134747 45.112547) (width 0.5) (layer "B.Cu") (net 7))
 (segment (start 89.518269 44.696651) (end 71.731632 44.696651) (width 0.5) (layer "B.Cu") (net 7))
 (segment (start 91.442147 45.493547) (end 91.600954 45.652354) (width 0.5) (layer "B.Cu") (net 7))
 (segment (start 125.745903 54.172998) (end 123.157251 56.761651) (width 0.5) (layer "B.Cu") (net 7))
 (segment (start 126.5428 52.24912) (end 126.5428 51.647581) (width 0.5) (layer "B.Cu") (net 7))
 (segment (start 97.655651 44.785551) (end 97.655651 44.315651) (width 0.5) (layer "B.Cu") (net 7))
 (segment (start 97.05875 45.85235) (end 97.323381 45.58772) (width 0.5) (layer "B.Cu") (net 7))
 (arc (start 97.655651 44.785551) (mid 97.569296 45.219681) (end 97.323381 45.58772) (width 0.5) (layer "B.Cu") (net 7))
 (arc (start 71.731632 44.696651) (mid 70.690437 44.903757) (end 69.807754 45.493547) (width 0.5) (layer "B.Cu") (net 7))
 (arc (start 121.134747 45.112547) (mid 120.252064 44.522757) (end 119.210869 44.315651) (width 0.5) (layer "B.Cu") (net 7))
 (arc (start 125.745903 49.723703) (mid 126.335693 50.606386) (end 126.5428 51.647581) (width 0.5) (layer "B.Cu") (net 7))
 (arc (start 91.600954 45.652354) (mid 92.483637 46.242144) (end 93.524832 46.449251) (width 0.5) (layer "B.Cu") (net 7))
 (arc (start 97.05875 45.85235) (mid 96.397593 46.294121) (end 95.617706 46.449251) (width 0.5) (layer "B.Cu") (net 7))
 (arc (start 91.442147 45.493547) (mid 90.559464 44.903757) (end 89.518269 44.696651) (width 0.5) (layer "B.Cu") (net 7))
 (arc (start 126.5428 52.24912) (mid 126.335693 53.290315) (end 125.745903 54.172998) (width 0.5) (layer "B.Cu") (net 7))
 (segment (start 123.157251 51.618151) (end 123.157251 51.554651) (width 0.5) (layer "F.Cu") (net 15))
 (segment (start 102.989651 49.141651) (end 110.219269 49.141651) (width 0.5) (layer "F.Cu") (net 15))
 (segment (start 70.833251 45.280851) (end 70.503051 45.611051) (width 0.5) (layer "F.Cu") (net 15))
 (segment (start 70.172851 46.408224) (end 70.172851 47.668451) (width 0.5) (layer "F.Cu") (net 15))
 (segment (start 100.678251 52.329351) (end 100.678251 53.205651) (width 0.25) (layer "F.Cu") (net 15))
 (segment (start 70.833251 45.280851) (end 67.896232 45.280851) (width 0.5) (layer "F.Cu") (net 15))
 (segment (start 102.989651 49.141651) (end 101.627547 47.779547) (width 0.5) (layer "F.Cu") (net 15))
 (segment (start 123.112349 51.726552) (end 122.522251 52.316651) (width 0.5) (layer "F.Cu") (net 15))
 (segment (start 99.703669 46.982651) (end 93.194632 46.982651) (width 0.5) (layer "F.Cu") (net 15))
 (segment (start 102.989651 49.141651) (end 101.297888 50.833413) (width 0.25) (layer "F.Cu") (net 15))
 (segment (start 115.156251 52.951651) (end 112.143147 49.938547) (width 0.5) (layer "F.Cu") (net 15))
 (segment (start 115.156251 52.951651) (end 120.989225 52.951651) (width 0.5) (layer "F.Cu") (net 15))
 (segment (start 91.162747 46.077747) (end 91.270754 46.185754) (width 0.5) (layer "F.Cu") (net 15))
 (segment (start 62.730651 50.446432) (end 62.730651 72.525669) (width 0.5) (layer "F.Cu") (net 15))
 (segment (start 70.833251 45.280851) (end 89.238869 45.280851) (width 0.5) (layer "F.Cu") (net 15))
 (segment (start 63.527547 74.449547) (end 65.143651 76.065651) (width 0.5) (layer "F.Cu") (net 15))
 (segment (start 63.527547 48.522554) (end 65.972354 46.077747) (width 0.5) (layer "F.Cu") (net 15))
 (arc (start 62.730651 72.525669) (mid 62.937757 73.566864) (end 63.527547 74.449547) (width 0.5) (layer "F.Cu") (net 15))
 (arc (start 67.896232 45.280851) (mid 66.855037 45.487957) (end 65.972354 46.077747) (width 0.5) (layer "F.Cu") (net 15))
 (arc (start 91.270754 46.185754) (mid 92.153437 46.775544) (end 93.194632 46.982651) (width 0.5) (layer "F.Cu") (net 15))
 (arc (start 63.527547 48.522554) (mid 62.937757 49.405237) (end 62.730651 50.446432) (width 0.5) (layer "F.Cu") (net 15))
 (arc (start 123.157251 51.618151) (mid 123.145581 51.676817) (end 123.112349 51.726552) (width 0.5) (layer "F.Cu") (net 15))
 (arc (start 122.522251 52.316651) (mid 121.818892 52.786619) (end 120.989225 52.951651) (width 0.5) (layer "F.Cu") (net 15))
 (arc (start 70.503051 45.611051) (mid 70.258667 45.976797) (end 70.172851 46.408224) (width 0.5) (layer "F.Cu") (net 15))
 (arc (start 101.297888 50.833413) (mid 100.839289 51.519755) (end 100.678251 52.329351) (width 0.25) (layer "F.Cu") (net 15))
 (arc (start 101.627547 47.779547) (mid 100.744864 47.189757) (end 99.703669 46.982651) (width 0.5) (layer "F.Cu") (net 15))
 (arc (start 91.162747 46.077747) (mid 90.280064 45.487957) (end 89.238869 45.280851) (width 0.5) (layer "F.Cu") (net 15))
 (arc (start 112.143147 49.938547) (mid 111.260464 49.348757) (end 110.219269 49.141651) (width 0.5) (layer "F.Cu") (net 15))
 (segment (start 102.456251 75.700669) (end 102.456251 56.110632) (width 0.25) (layer "B.Cu") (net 15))
 (segment (start 101.659354 77.624547) (end 100.678251 78.605651) (width 0.25) (layer "B.Cu") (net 15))
 (segment (start 101.659354 54.186754) (end 100.678251 53.205651) (width 0.25) (layer "B.Cu") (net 15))
 (arc (start 101.659354 54.186754) (mid 102.249144 55.069437) (end 102.456251 56.110632) (width 0.25) (layer "B.Cu") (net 15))
 (arc (start 102.456251 75.700669) (mid 102.249144 76.741864) (end 101.659354 77.624547) (width 0.25) (layer "B.Cu") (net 15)))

